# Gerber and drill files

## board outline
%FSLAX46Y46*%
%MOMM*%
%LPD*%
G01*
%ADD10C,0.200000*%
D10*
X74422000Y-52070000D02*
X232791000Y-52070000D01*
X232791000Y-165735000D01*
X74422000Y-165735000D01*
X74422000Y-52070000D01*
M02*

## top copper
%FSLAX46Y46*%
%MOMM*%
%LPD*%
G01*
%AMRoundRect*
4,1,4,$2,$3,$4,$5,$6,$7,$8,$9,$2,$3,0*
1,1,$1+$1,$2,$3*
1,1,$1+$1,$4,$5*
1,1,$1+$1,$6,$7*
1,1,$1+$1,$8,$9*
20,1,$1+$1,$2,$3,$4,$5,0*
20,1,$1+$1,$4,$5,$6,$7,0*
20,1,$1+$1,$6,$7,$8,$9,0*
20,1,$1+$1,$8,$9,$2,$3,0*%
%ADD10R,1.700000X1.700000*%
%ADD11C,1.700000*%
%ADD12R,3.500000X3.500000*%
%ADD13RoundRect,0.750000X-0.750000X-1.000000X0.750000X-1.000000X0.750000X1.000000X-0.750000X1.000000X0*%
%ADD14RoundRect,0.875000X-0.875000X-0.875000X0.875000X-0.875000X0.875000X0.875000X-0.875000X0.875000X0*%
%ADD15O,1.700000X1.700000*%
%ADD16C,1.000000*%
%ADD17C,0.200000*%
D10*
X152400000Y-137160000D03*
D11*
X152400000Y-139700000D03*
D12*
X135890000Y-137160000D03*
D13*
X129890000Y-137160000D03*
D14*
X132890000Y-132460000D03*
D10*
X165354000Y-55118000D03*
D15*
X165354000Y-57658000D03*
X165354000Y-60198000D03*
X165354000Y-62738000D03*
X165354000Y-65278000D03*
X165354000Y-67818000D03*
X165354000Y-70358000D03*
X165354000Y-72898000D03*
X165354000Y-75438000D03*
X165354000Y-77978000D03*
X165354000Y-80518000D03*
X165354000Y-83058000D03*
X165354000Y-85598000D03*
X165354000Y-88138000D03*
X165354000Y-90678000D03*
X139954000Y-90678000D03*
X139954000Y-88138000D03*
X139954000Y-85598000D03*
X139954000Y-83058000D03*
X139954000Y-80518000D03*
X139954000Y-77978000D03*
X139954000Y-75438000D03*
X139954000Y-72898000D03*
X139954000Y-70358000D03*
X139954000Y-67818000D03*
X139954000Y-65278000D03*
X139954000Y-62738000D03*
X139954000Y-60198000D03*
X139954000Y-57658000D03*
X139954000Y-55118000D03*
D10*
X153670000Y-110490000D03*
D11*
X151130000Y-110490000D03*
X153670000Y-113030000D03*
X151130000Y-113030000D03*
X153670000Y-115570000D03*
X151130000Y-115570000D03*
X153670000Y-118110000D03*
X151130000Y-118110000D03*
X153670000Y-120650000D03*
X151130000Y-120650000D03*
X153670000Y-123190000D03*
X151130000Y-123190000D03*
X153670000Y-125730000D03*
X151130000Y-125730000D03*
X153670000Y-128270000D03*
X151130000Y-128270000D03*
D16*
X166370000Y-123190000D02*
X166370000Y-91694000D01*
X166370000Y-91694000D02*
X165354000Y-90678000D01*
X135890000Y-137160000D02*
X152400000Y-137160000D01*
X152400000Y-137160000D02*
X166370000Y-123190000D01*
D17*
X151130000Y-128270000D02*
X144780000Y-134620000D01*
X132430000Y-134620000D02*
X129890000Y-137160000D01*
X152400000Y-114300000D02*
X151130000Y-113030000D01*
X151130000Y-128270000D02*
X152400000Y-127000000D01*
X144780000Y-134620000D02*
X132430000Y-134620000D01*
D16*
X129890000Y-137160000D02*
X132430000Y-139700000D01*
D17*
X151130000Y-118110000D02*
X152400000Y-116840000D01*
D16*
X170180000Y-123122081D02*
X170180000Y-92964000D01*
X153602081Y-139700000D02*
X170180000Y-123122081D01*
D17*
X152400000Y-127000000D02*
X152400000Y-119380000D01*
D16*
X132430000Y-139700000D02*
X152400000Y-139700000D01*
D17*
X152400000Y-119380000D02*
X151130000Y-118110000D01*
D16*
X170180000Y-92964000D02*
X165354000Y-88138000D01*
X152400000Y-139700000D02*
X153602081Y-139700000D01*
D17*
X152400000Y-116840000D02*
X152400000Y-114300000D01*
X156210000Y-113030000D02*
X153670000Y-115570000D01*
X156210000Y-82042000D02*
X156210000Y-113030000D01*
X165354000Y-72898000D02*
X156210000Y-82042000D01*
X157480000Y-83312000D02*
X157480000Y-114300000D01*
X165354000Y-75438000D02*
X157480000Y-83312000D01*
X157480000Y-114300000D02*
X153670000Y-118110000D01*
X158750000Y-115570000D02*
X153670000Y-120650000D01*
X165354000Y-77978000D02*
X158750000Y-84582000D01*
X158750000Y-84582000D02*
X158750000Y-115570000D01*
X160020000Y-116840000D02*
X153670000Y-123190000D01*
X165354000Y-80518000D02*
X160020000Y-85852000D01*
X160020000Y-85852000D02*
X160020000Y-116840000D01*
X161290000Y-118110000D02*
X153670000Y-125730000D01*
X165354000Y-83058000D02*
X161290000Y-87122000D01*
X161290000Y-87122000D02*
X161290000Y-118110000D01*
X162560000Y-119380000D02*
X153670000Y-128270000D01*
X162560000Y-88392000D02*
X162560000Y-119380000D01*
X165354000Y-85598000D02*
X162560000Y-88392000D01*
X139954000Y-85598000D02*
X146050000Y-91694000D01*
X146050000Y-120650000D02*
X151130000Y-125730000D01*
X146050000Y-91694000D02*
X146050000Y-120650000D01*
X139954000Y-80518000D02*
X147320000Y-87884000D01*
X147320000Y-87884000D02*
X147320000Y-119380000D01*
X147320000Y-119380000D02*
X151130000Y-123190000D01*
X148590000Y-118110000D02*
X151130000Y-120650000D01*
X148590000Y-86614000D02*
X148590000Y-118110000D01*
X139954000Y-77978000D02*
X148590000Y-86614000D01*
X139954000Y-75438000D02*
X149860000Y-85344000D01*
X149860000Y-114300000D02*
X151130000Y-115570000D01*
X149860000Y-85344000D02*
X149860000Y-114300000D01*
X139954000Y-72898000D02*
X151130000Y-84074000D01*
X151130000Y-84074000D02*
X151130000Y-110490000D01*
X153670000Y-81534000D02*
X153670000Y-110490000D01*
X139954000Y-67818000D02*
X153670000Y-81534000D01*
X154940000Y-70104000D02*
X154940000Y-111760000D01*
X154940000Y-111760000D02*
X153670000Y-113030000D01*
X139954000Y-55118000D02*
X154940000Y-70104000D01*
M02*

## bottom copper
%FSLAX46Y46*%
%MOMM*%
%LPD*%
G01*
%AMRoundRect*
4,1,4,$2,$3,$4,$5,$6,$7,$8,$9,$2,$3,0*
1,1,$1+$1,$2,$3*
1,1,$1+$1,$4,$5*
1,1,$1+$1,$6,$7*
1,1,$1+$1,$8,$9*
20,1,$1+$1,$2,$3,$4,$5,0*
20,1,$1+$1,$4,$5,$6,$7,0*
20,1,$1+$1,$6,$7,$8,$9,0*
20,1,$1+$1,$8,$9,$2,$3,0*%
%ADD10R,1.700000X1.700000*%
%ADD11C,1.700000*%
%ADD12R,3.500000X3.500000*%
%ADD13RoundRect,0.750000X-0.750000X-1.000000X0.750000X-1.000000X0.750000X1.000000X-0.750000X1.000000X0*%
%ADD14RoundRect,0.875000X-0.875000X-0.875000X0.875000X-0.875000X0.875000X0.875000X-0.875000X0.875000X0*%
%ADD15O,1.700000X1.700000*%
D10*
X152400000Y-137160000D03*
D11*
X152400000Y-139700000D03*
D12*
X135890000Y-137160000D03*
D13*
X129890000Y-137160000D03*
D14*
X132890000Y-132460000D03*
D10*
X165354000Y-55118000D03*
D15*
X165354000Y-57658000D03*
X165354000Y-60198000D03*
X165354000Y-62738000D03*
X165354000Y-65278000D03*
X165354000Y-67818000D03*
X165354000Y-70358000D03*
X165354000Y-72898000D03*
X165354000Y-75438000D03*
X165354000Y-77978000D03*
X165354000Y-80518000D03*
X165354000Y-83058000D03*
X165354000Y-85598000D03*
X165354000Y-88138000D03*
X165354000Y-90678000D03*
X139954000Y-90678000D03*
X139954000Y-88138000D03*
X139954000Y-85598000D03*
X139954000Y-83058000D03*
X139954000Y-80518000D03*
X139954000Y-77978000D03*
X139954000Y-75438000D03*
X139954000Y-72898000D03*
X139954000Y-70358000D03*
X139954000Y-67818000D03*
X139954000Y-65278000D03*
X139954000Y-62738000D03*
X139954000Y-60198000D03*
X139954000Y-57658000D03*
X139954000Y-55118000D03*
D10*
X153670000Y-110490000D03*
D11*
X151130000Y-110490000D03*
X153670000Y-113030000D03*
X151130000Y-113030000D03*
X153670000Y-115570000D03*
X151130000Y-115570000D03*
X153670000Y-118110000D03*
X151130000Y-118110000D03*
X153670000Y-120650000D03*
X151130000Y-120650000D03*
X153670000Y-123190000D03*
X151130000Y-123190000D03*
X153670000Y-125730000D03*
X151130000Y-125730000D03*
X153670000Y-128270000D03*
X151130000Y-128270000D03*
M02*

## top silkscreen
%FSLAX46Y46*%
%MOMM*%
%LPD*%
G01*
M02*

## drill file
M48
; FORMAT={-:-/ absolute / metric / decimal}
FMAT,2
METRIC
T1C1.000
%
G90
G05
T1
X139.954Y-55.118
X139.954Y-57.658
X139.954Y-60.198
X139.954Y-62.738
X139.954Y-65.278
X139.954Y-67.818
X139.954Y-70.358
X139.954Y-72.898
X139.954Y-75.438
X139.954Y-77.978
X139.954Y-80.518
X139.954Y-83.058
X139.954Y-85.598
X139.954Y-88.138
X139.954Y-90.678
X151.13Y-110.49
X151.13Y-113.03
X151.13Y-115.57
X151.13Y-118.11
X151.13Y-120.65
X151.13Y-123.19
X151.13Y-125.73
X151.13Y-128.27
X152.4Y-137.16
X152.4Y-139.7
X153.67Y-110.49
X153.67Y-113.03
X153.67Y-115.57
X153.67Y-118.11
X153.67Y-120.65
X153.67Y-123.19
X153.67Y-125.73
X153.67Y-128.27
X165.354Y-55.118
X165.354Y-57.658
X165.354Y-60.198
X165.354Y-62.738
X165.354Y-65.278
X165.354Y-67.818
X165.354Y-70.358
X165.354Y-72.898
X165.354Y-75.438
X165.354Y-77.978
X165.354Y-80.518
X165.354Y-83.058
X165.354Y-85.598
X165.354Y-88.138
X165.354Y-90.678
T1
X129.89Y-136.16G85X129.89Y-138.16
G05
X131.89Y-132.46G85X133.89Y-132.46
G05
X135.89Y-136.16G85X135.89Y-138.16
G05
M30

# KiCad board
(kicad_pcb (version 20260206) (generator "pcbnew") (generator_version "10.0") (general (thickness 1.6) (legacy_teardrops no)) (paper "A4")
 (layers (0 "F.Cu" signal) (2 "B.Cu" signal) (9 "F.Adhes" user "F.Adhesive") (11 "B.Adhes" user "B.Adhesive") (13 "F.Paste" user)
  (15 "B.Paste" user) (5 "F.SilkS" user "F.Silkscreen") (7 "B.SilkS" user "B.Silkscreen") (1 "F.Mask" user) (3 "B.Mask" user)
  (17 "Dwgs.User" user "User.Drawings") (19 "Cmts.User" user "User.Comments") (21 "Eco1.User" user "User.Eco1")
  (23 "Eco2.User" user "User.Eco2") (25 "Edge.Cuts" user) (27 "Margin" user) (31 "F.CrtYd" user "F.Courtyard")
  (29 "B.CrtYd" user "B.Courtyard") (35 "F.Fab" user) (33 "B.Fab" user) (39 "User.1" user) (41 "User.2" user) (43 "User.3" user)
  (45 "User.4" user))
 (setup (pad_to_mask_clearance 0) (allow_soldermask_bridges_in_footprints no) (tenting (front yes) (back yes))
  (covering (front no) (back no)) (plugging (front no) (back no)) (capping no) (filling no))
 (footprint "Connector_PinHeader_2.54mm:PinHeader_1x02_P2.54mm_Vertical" (layer "B.Cu") (at 152.4 137.16 180)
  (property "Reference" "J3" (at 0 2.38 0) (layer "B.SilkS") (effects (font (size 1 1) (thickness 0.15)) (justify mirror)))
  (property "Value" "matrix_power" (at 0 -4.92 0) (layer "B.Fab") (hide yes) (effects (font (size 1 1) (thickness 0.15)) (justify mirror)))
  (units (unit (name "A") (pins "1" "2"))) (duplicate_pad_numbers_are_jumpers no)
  (pad "1" thru_hole rect (at 0 0 180) (size 1.7 1.7) (drill 1) (layers "*.Cu" "*.Mask") (remove_unused_layers no) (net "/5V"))
  (pad "2" thru_hole circle (at 0 -2.54 180) (size 1.7 1.7) (drill 1) (layers "*.Cu" "*.Mask") (remove_unused_layers no) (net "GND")))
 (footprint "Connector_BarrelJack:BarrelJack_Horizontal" (layer "B.Cu") (at 135.89 137.16)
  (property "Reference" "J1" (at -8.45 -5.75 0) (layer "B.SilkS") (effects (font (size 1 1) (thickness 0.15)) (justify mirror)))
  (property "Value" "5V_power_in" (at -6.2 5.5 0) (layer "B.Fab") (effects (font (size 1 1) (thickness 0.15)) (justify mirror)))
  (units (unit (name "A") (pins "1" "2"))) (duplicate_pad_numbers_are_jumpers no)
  (pad "1" thru_hole rect (at 0 0) (size 3.5 3.5) (drill oval 1 3) (layers "*.Cu" "*.Mask") (remove_unused_layers no) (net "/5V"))
  (pad "2" thru_hole roundrect (at -6 0) (size 3 3.5) (drill oval 1 3) (layers "*.Cu" "*.Mask") (remove_unused_layers no)
   (roundrect_rratio 0.25) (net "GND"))
  (pad "3" thru_hole roundrect (at -3 -4.7) (size 3.5 3.5) (drill oval 3 1) (layers "*.Cu" "*.Mask") (remove_unused_layers no)
   (roundrect_rratio 0.25)))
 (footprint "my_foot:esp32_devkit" (layer "B.Cu") (at 165.354 55.118 180)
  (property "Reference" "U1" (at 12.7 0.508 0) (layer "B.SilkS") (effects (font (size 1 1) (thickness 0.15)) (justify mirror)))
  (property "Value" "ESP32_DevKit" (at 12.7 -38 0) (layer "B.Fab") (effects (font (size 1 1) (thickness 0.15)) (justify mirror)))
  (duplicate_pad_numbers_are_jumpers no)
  (pad "1" thru_hole rect (at 0 0 180) (size 1.7 1.7) (drill 1) (layers "*.Cu" "*.Mask") (remove_unused_layers no)
   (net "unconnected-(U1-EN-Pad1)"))
  (pad "2" thru_hole oval (at 0 -2.54 180) (size 1.7 1.7) (drill 1) (layers "*.Cu" "*.Mask") (remove_unused_layers no)
   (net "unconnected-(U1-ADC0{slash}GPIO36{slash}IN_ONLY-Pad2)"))
  (pad "3" thru_hole oval (at 0 -5.08 180) (size 1.7 1.7) (drill 1) (layers "*.Cu" "*.Mask") (remove_unused_layers no)
   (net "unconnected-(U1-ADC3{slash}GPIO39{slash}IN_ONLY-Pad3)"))
  (pad "4" thru_hole oval (at 0 -7.62 180) (size 1.7 1.7) (drill 1) (layers "*.Cu" "*.Mask") (remove_unused_layers no)
   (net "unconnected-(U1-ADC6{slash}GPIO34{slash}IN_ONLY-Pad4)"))
  (pad "5" thru_hole oval (at 0 -10.16 180) (size 1.7 1.7) (drill 1) (layers "*.Cu" "*.Mask") (remove_unused_layers no)
   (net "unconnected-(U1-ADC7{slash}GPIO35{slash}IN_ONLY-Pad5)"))
  (pad "6" thru_hole oval (at 0 -12.7 180) (size 1.7 1.7) (drill 1) (layers "*.Cu" "*.Mask") (remove_unused_layers no)
   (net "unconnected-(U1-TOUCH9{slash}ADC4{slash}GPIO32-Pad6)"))
  (pad "7" thru_hole oval (at 0 -15.24 180) (size 1.7 1.7) (drill 1) (layers "*.Cu" "*.Mask") (remove_unused_layers no)
   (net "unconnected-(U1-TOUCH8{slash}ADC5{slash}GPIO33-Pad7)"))
  (pad "8" thru_hole oval (at 0 -17.78 180) (size 1.7 1.7) (drill 1) (layers "*.Cu" "*.Mask") (remove_unused_layers no) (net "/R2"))
  (pad "9" thru_hole oval (at 0 -20.32 180) (size 1.7 1.7) (drill 1) (layers "*.Cu" "*.Mask") (remove_unused_layers no) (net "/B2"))
  (pad "10" thru_hole oval (at 0 -22.86 180) (size 1.7 1.7) (drill 1) (layers "*.Cu" "*.Mask") (remove_unused_layers no) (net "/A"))
  (pad "11" thru_hole oval (at 0 -25.4 180) (size 1.7 1.7) (drill 1) (layers "*.Cu" "*.Mask") (remove_unused_layers no) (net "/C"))
  (pad "12" thru_hole oval (at 0 -27.94 180) (size 1.7 1.7) (drill 1) (layers "*.Cu" "*.Mask") (remove_unused_layers no) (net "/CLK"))
  (pad "13" thru_hole oval (at 0 -30.48 180) (size 1.7 1.7) (drill 1) (layers "*.Cu" "*.Mask") (remove_unused_layers no) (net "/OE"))
  (pad "14" thru_hole oval (at 0 -33.02 180) (size 1.7 1.7) (drill 1) (layers "*.Cu" "*.Mask") (remove_unused_layers no) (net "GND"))
  (pad "15" thru_hole oval (at 0 -35.56 180) (size 1.7 1.7) (drill 1) (layers "*.Cu" "*.Mask") (remove_unused_layers no) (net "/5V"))
  (pad "16" thru_hole oval (at 25.4 -35.56 180) (size 1.7 1.7) (drill 1) (layers "*.Cu" "*.Mask") (remove_unused_layers no)
   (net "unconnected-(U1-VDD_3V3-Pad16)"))
  (pad "17" thru_hole oval (at 25.4 -33.02 180) (size 1.7 1.7) (drill 1) (layers "*.Cu" "*.Mask") (remove_unused_layers no)
   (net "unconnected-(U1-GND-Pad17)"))
  (pad "18" thru_hole oval (at 25.4 -30.48 180) (size 1.7 1.7) (drill 1) (layers "*.Cu" "*.Mask") (remove_unused_layers no) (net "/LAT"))
  (pad "19" thru_hole oval (at 25.4 -27.94 180) (size 1.7 1.7) (drill 1) (layers "*.Cu" "*.Mask") (remove_unused_layers no)
   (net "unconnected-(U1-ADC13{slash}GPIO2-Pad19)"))
  (pad "20" thru_hole oval (at 25.4 -25.4 180) (size 1.7 1.7) (drill 1) (layers "*.Cu" "*.Mask") (remove_unused_layers no) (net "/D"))
  (pad "21" thru_hole oval (at 25.4 -22.86 180) (size 1.7 1.7) (drill 1) (layers "*.Cu" "*.Mask") (remove_unused_layers no) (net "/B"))
  (pad "22" thru_hole oval (at 25.4 -20.32 180) (size 1.7 1.7) (drill 1) (layers "*.Cu" "*.Mask") (remove_unused_layers no) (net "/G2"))
  (pad "23" thru_hole oval (at 25.4 -17.78 180) (size 1.7 1.7) (drill 1) (layers "*.Cu" "*.Mask") (remove_unused_layers no) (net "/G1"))
  (pad "24" thru_hole oval (at 25.4 -15.24 180) (size 1.7 1.7) (drill 1) (layers "*.Cu" "*.Mask") (remove_unused_layers no)
   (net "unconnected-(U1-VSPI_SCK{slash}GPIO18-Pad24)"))
  (pad "25" thru_hole oval (at 25.4 -12.7 180) (size 1.7 1.7) (drill 1) (layers "*.Cu" "*.Mask") (remove_unused_layers no) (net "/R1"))
  (pad "26" thru_hole oval (at 25.4 -10.16 180) (size 1.7 1.7) (drill 1) (layers "*.Cu" "*.Mask") (remove_unused_layers no)
   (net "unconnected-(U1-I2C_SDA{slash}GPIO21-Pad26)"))
  (pad "27" thru_hole oval (at 25.4 -7.62 180) (size 1.7 1.7) (drill 1) (layers "*.Cu" "*.Mask") (remove_unused_layers no)
   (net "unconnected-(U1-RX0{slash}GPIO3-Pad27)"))
  (pad "28" thru_hole oval (at 25.4 -5.08 180) (size 1.7 1.7) (drill 1) (layers "*.Cu" "*.Mask") (remove_unused_layers no)
   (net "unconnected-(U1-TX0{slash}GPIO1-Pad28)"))
  (pad "29" thru_hole oval (at 25.4 -2.54 180) (size 1.7 1.7) (drill 1) (layers "*.Cu" "*.Mask") (remove_unused_layers no)
   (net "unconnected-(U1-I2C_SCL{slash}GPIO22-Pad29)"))
  (pad "30" thru_hole oval (at 25.4 0 180) (size 1.7 1.7) (drill 1) (layers "*.Cu" "*.Mask") (remove_unused_layers no) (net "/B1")))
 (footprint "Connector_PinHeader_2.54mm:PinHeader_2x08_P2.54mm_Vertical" (layer "B.Cu") (at 153.67 110.49 180)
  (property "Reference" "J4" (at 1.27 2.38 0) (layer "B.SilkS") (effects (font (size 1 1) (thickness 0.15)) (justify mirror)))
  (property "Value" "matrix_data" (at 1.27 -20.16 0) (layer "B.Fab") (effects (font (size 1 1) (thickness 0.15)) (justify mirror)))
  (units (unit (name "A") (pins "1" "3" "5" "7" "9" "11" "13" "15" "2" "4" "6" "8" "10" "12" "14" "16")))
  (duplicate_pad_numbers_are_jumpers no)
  (pad "1" thru_hole rect (at 0 0 180) (size 1.7 1.7) (drill 1) (layers "*.Cu" "*.Mask") (remove_unused_layers no) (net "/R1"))
  (pad "2" thru_hole circle (at 2.54 0 180) (size 1.7 1.7) (drill 1) (layers "*.Cu" "*.Mask") (remove_unused_layers no) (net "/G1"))
  (pad "3" thru_hole circle (at 0 -2.54 180) (size 1.7 1.7) (drill 1) (layers "*.Cu" "*.Mask") (remove_unused_layers no) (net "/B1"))
  (pad "4" thru_hole circle (at 2.54 -2.54 180) (size 1.7 1.7) (drill 1) (layers "*.Cu" "*.Mask") (remove_unused_layers no) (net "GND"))
  (pad "5" thru_hole circle (at 0 -5.08 180) (size 1.7 1.7) (drill 1) (layers "*.Cu" "*.Mask") (remove_unused_layers no) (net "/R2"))
  (pad "6" thru_hole circle (at 2.54 -5.08 180) (size 1.7 1.7) (drill 1) (layers "*.Cu" "*.Mask") (remove_unused_layers no) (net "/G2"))
  (pad "7" thru_hole circle (at 0 -7.62 180) (size 1.7 1.7) (drill 1) (layers "*.Cu" "*.Mask") (remove_unused_layers no) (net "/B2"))
  (pad "8" thru_hole circle (at 2.54 -7.62 180) (size 1.7 1.7) (drill 1) (layers "*.Cu" "*.Mask") (remove_unused_layers no) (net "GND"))
  (pad "9" thru_hole circle (at 0 -10.16 180) (size 1.7 1.7) (drill 1) (layers "*.Cu" "*.Mask") (remove_unused_layers no) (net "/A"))
  (pad "10" thru_hole circle (at 2.54 -10.16 180) (size 1.7 1.7) (drill 1) (layers "*.Cu" "*.Mask") (remove_unused_layers no) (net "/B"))
  (pad "11" thru_hole circle (at 0 -12.7 180) (size 1.7 1.7) (drill 1) (layers "*.Cu" "*.Mask") (remove_unused_layers no) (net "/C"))
  (pad "12" thru_hole circle (at 2.54 -12.7 180) (size 1.7 1.7) (drill 1) (layers "*.Cu" "*.Mask") (remove_unused_layers no) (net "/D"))
  (pad "13" thru_hole circle (at 0 -15.24 180) (size 1.7 1.7) (drill 1) (layers "*.Cu" "*.Mask") (remove_unused_layers no) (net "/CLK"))
  (pad "14" thru_hole circle (at 2.54 -15.24 180) (size 1.7 1.7) (drill 1) (layers "*.Cu" "*.Mask") (remove_unused_layers no) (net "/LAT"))
  (pad "15" thru_hole circle (at 0 -17.78 180) (size 1.7 1.7) (drill 1) (layers "*.Cu" "*.Mask") (remove_unused_layers no) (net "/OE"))
  (pad "16" thru_hole circle (at 2.54 -17.78 180) (size 1.7 1.7) (drill 1) (layers "*.Cu" "*.Mask") (remove_unused_layers no) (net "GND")))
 (gr_rect (start 74.422 52.07) (end 232.791 165.735) (stroke (width 0.2) (type solid)) (fill no) (layer "Edge.Cuts"))
 (segment (start 166.37 123.19) (end 166.37 91.694) (width 1) (layer "F.Cu") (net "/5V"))
 (segment (start 166.37 91.694) (end 165.354 90.678) (width 1) (layer "F.Cu") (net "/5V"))
 (segment (start 135.89 137.16) (end 152.4 137.16) (width 1) (layer "F.Cu") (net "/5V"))
 (segment (start 152.4 137.16) (end 166.37 123.19) (width 1) (layer "F.Cu") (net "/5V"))
 (segment (start 151.13 128.27) (end 144.78 134.62) (width 0.2) (layer "F.Cu") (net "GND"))
 (segment (start 132.43 134.62) (end 129.89 137.16) (width 0.2) (layer "F.Cu") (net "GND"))
 (segment (start 152.4 114.3) (end 151.13 113.03) (width 0.2) (layer "F.Cu") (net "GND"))
 (segment (start 151.13 128.27) (end 152.4 127) (width 0.2) (layer "F.Cu") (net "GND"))
 (segment (start 144.78 134.62) (end 132.43 134.62) (width 0.2) (layer "F.Cu") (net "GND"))
 (segment (start 129.89 137.16) (end 132.43 139.7) (width 1) (layer "F.Cu") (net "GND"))
 (segment (start 151.13 118.11) (end 152.4 116.84) (width 0.2) (layer "F.Cu") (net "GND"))
 (segment (start 170.18 123.122081) (end 170.18 92.964) (width 1) (layer "F.Cu") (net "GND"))
 (segment (start 153.602081 139.7) (end 170.18 123.122081) (width 1) (layer "F.Cu") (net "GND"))
 (segment (start 152.4 127) (end 152.4 119.38) (width 0.2) (layer "F.Cu") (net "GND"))
 (segment (start 132.43 139.7) (end 152.4 139.7) (width 1) (layer "F.Cu") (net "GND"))
 (segment (start 152.4 119.38) (end 151.13 118.11) (width 0.2) (layer "F.Cu") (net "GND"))
 (segment (start 170.18 92.964) (end 165.354 88.138) (width 1) (layer "F.Cu") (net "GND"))
 (segment (start 152.4 139.7) (end 153.602081 139.7) (width 1) (layer "F.Cu") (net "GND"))
 (segment (start 152.4 116.84) (end 152.4 114.3) (width 0.2) (layer "F.Cu") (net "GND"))
 (segment (start 156.21 113.03) (end 153.67 115.57) (width 0.2) (layer "F.Cu") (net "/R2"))
 (segment (start 156.21 82.042) (end 156.21 113.03) (width 0.2) (layer "F.Cu") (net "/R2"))
 (segment (start 165.354 72.898) (end 156.21 82.042) (width 0.2) (layer "F.Cu") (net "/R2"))
 (segment (start 157.48 83.312) (end 157.48 114.3) (width 0.2) (layer "F.Cu") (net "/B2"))
 (segment (start 165.354 75.438) (end 157.48 83.312) (width 0.2) (layer "F.Cu") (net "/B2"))
 (segment (start 157.48 114.3) (end 153.67 118.11) (width 0.2) (layer "F.Cu") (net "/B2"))
 (segment (start 158.75 115.57) (end 153.67 120.65) (width 0.2) (layer "F.Cu") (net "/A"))
 (segment (start 165.354 77.978) (end 158.75 84.582) (width 0.2) (layer "F.Cu") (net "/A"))
 (segment (start 158.75 84.582) (end 158.75 115.57) (width 0.2) (layer "F.Cu") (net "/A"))
 (segment (start 160.02 116.84) (end 153.67 123.19) (width 0.2) (layer "F.Cu") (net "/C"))
 (segment (start 165.354 80.518) (end 160.02 85.852) (width 0.2) (layer "F.Cu") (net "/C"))
 (segment (start 160.02 85.852) (end 160.02 116.84) (width 0.2) (layer "F.Cu") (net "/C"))
 (segment (start 161.29 118.11) (end 153.67 125.73) (width 0.2) (layer "F.Cu") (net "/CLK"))
 (segment (start 165.354 83.058) (end 161.29 87.122) (width 0.2) (layer "F.Cu") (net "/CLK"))
 (segment (start 161.29 87.122) (end 161.29 118.11) (width 0.2) (layer "F.Cu") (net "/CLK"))
 (segment (start 162.56 119.38) (end 153.67 128.27) (width 0.2) (layer "F.Cu") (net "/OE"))
 (segment (start 162.56 88.392) (end 162.56 119.38) (width 0.2) (layer "F.Cu") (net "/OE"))
 (segment (start 165.354 85.598) (end 162.56 88.392) (width 0.2) (layer "F.Cu") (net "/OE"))
 (segment (start 139.954 85.598) (end 146.05 91.694) (width 0.2) (layer "F.Cu") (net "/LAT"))
 (segment (start 146.05 120.65) (end 151.13 125.73) (width 0.2) (layer "F.Cu") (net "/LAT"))
 (segment (start 146.05 91.694) (end 146.05 120.65) (width 0.2) (layer "F.Cu") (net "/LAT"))
 (segment (start 139.954 80.518) (end 147.32 87.884) (width 0.2) (layer "F.Cu") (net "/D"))
 (segment (start 147.32 87.884) (end 147.32 119.38) (width 0.2) (layer "F.Cu") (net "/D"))
 (segment (start 147.32 119.38) (end 151.13 123.19) (width 0.2) (layer "F.Cu") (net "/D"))
 (segment (start 148.59 118.11) (end 151.13 120.65) (width 0.2) (layer "F.Cu") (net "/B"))
 (segment (start 148.59 86.614) (end 148.59 118.11) (width 0.2) (layer "F.Cu") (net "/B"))
 (segment (start 139.954 77.978) (end 148.59 86.614) (width 0.2) (layer "F.Cu") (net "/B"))
 (segment (start 139.954 75.438) (end 149.86 85.344) (width 0.2) (layer "F.Cu") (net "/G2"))
 (segment (start 149.86 114.3) (end 151.13 115.57) (width 0.2) (layer "F.Cu") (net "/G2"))
 (segment (start 149.86 85.344) (end 149.86 114.3) (width 0.2) (layer "F.Cu") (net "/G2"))
 (segment (start 139.954 72.898) (end 151.13 84.074) (width 0.2) (layer "F.Cu") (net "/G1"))
 (segment (start 151.13 84.074) (end 151.13 110.49) (width 0.2) (layer "F.Cu") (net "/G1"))
 (segment (start 153.67 81.534) (end 153.67 110.49) (width 0.2) (layer "F.Cu") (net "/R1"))
 (segment (start 139.954 67.818) (end 153.67 81.534) (width 0.2) (layer "F.Cu") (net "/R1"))
 (segment (start 154.94 70.104) (end 154.94 111.76) (width 0.2) (layer "F.Cu") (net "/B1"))
 (segment (start 154.94 111.76) (end 153.67 113.03) (width 0.2) (layer "F.Cu") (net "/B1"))
 (segment (start 139.954 55.118) (end 154.94 70.104) (width 0.2) (layer "F.Cu") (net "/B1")))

